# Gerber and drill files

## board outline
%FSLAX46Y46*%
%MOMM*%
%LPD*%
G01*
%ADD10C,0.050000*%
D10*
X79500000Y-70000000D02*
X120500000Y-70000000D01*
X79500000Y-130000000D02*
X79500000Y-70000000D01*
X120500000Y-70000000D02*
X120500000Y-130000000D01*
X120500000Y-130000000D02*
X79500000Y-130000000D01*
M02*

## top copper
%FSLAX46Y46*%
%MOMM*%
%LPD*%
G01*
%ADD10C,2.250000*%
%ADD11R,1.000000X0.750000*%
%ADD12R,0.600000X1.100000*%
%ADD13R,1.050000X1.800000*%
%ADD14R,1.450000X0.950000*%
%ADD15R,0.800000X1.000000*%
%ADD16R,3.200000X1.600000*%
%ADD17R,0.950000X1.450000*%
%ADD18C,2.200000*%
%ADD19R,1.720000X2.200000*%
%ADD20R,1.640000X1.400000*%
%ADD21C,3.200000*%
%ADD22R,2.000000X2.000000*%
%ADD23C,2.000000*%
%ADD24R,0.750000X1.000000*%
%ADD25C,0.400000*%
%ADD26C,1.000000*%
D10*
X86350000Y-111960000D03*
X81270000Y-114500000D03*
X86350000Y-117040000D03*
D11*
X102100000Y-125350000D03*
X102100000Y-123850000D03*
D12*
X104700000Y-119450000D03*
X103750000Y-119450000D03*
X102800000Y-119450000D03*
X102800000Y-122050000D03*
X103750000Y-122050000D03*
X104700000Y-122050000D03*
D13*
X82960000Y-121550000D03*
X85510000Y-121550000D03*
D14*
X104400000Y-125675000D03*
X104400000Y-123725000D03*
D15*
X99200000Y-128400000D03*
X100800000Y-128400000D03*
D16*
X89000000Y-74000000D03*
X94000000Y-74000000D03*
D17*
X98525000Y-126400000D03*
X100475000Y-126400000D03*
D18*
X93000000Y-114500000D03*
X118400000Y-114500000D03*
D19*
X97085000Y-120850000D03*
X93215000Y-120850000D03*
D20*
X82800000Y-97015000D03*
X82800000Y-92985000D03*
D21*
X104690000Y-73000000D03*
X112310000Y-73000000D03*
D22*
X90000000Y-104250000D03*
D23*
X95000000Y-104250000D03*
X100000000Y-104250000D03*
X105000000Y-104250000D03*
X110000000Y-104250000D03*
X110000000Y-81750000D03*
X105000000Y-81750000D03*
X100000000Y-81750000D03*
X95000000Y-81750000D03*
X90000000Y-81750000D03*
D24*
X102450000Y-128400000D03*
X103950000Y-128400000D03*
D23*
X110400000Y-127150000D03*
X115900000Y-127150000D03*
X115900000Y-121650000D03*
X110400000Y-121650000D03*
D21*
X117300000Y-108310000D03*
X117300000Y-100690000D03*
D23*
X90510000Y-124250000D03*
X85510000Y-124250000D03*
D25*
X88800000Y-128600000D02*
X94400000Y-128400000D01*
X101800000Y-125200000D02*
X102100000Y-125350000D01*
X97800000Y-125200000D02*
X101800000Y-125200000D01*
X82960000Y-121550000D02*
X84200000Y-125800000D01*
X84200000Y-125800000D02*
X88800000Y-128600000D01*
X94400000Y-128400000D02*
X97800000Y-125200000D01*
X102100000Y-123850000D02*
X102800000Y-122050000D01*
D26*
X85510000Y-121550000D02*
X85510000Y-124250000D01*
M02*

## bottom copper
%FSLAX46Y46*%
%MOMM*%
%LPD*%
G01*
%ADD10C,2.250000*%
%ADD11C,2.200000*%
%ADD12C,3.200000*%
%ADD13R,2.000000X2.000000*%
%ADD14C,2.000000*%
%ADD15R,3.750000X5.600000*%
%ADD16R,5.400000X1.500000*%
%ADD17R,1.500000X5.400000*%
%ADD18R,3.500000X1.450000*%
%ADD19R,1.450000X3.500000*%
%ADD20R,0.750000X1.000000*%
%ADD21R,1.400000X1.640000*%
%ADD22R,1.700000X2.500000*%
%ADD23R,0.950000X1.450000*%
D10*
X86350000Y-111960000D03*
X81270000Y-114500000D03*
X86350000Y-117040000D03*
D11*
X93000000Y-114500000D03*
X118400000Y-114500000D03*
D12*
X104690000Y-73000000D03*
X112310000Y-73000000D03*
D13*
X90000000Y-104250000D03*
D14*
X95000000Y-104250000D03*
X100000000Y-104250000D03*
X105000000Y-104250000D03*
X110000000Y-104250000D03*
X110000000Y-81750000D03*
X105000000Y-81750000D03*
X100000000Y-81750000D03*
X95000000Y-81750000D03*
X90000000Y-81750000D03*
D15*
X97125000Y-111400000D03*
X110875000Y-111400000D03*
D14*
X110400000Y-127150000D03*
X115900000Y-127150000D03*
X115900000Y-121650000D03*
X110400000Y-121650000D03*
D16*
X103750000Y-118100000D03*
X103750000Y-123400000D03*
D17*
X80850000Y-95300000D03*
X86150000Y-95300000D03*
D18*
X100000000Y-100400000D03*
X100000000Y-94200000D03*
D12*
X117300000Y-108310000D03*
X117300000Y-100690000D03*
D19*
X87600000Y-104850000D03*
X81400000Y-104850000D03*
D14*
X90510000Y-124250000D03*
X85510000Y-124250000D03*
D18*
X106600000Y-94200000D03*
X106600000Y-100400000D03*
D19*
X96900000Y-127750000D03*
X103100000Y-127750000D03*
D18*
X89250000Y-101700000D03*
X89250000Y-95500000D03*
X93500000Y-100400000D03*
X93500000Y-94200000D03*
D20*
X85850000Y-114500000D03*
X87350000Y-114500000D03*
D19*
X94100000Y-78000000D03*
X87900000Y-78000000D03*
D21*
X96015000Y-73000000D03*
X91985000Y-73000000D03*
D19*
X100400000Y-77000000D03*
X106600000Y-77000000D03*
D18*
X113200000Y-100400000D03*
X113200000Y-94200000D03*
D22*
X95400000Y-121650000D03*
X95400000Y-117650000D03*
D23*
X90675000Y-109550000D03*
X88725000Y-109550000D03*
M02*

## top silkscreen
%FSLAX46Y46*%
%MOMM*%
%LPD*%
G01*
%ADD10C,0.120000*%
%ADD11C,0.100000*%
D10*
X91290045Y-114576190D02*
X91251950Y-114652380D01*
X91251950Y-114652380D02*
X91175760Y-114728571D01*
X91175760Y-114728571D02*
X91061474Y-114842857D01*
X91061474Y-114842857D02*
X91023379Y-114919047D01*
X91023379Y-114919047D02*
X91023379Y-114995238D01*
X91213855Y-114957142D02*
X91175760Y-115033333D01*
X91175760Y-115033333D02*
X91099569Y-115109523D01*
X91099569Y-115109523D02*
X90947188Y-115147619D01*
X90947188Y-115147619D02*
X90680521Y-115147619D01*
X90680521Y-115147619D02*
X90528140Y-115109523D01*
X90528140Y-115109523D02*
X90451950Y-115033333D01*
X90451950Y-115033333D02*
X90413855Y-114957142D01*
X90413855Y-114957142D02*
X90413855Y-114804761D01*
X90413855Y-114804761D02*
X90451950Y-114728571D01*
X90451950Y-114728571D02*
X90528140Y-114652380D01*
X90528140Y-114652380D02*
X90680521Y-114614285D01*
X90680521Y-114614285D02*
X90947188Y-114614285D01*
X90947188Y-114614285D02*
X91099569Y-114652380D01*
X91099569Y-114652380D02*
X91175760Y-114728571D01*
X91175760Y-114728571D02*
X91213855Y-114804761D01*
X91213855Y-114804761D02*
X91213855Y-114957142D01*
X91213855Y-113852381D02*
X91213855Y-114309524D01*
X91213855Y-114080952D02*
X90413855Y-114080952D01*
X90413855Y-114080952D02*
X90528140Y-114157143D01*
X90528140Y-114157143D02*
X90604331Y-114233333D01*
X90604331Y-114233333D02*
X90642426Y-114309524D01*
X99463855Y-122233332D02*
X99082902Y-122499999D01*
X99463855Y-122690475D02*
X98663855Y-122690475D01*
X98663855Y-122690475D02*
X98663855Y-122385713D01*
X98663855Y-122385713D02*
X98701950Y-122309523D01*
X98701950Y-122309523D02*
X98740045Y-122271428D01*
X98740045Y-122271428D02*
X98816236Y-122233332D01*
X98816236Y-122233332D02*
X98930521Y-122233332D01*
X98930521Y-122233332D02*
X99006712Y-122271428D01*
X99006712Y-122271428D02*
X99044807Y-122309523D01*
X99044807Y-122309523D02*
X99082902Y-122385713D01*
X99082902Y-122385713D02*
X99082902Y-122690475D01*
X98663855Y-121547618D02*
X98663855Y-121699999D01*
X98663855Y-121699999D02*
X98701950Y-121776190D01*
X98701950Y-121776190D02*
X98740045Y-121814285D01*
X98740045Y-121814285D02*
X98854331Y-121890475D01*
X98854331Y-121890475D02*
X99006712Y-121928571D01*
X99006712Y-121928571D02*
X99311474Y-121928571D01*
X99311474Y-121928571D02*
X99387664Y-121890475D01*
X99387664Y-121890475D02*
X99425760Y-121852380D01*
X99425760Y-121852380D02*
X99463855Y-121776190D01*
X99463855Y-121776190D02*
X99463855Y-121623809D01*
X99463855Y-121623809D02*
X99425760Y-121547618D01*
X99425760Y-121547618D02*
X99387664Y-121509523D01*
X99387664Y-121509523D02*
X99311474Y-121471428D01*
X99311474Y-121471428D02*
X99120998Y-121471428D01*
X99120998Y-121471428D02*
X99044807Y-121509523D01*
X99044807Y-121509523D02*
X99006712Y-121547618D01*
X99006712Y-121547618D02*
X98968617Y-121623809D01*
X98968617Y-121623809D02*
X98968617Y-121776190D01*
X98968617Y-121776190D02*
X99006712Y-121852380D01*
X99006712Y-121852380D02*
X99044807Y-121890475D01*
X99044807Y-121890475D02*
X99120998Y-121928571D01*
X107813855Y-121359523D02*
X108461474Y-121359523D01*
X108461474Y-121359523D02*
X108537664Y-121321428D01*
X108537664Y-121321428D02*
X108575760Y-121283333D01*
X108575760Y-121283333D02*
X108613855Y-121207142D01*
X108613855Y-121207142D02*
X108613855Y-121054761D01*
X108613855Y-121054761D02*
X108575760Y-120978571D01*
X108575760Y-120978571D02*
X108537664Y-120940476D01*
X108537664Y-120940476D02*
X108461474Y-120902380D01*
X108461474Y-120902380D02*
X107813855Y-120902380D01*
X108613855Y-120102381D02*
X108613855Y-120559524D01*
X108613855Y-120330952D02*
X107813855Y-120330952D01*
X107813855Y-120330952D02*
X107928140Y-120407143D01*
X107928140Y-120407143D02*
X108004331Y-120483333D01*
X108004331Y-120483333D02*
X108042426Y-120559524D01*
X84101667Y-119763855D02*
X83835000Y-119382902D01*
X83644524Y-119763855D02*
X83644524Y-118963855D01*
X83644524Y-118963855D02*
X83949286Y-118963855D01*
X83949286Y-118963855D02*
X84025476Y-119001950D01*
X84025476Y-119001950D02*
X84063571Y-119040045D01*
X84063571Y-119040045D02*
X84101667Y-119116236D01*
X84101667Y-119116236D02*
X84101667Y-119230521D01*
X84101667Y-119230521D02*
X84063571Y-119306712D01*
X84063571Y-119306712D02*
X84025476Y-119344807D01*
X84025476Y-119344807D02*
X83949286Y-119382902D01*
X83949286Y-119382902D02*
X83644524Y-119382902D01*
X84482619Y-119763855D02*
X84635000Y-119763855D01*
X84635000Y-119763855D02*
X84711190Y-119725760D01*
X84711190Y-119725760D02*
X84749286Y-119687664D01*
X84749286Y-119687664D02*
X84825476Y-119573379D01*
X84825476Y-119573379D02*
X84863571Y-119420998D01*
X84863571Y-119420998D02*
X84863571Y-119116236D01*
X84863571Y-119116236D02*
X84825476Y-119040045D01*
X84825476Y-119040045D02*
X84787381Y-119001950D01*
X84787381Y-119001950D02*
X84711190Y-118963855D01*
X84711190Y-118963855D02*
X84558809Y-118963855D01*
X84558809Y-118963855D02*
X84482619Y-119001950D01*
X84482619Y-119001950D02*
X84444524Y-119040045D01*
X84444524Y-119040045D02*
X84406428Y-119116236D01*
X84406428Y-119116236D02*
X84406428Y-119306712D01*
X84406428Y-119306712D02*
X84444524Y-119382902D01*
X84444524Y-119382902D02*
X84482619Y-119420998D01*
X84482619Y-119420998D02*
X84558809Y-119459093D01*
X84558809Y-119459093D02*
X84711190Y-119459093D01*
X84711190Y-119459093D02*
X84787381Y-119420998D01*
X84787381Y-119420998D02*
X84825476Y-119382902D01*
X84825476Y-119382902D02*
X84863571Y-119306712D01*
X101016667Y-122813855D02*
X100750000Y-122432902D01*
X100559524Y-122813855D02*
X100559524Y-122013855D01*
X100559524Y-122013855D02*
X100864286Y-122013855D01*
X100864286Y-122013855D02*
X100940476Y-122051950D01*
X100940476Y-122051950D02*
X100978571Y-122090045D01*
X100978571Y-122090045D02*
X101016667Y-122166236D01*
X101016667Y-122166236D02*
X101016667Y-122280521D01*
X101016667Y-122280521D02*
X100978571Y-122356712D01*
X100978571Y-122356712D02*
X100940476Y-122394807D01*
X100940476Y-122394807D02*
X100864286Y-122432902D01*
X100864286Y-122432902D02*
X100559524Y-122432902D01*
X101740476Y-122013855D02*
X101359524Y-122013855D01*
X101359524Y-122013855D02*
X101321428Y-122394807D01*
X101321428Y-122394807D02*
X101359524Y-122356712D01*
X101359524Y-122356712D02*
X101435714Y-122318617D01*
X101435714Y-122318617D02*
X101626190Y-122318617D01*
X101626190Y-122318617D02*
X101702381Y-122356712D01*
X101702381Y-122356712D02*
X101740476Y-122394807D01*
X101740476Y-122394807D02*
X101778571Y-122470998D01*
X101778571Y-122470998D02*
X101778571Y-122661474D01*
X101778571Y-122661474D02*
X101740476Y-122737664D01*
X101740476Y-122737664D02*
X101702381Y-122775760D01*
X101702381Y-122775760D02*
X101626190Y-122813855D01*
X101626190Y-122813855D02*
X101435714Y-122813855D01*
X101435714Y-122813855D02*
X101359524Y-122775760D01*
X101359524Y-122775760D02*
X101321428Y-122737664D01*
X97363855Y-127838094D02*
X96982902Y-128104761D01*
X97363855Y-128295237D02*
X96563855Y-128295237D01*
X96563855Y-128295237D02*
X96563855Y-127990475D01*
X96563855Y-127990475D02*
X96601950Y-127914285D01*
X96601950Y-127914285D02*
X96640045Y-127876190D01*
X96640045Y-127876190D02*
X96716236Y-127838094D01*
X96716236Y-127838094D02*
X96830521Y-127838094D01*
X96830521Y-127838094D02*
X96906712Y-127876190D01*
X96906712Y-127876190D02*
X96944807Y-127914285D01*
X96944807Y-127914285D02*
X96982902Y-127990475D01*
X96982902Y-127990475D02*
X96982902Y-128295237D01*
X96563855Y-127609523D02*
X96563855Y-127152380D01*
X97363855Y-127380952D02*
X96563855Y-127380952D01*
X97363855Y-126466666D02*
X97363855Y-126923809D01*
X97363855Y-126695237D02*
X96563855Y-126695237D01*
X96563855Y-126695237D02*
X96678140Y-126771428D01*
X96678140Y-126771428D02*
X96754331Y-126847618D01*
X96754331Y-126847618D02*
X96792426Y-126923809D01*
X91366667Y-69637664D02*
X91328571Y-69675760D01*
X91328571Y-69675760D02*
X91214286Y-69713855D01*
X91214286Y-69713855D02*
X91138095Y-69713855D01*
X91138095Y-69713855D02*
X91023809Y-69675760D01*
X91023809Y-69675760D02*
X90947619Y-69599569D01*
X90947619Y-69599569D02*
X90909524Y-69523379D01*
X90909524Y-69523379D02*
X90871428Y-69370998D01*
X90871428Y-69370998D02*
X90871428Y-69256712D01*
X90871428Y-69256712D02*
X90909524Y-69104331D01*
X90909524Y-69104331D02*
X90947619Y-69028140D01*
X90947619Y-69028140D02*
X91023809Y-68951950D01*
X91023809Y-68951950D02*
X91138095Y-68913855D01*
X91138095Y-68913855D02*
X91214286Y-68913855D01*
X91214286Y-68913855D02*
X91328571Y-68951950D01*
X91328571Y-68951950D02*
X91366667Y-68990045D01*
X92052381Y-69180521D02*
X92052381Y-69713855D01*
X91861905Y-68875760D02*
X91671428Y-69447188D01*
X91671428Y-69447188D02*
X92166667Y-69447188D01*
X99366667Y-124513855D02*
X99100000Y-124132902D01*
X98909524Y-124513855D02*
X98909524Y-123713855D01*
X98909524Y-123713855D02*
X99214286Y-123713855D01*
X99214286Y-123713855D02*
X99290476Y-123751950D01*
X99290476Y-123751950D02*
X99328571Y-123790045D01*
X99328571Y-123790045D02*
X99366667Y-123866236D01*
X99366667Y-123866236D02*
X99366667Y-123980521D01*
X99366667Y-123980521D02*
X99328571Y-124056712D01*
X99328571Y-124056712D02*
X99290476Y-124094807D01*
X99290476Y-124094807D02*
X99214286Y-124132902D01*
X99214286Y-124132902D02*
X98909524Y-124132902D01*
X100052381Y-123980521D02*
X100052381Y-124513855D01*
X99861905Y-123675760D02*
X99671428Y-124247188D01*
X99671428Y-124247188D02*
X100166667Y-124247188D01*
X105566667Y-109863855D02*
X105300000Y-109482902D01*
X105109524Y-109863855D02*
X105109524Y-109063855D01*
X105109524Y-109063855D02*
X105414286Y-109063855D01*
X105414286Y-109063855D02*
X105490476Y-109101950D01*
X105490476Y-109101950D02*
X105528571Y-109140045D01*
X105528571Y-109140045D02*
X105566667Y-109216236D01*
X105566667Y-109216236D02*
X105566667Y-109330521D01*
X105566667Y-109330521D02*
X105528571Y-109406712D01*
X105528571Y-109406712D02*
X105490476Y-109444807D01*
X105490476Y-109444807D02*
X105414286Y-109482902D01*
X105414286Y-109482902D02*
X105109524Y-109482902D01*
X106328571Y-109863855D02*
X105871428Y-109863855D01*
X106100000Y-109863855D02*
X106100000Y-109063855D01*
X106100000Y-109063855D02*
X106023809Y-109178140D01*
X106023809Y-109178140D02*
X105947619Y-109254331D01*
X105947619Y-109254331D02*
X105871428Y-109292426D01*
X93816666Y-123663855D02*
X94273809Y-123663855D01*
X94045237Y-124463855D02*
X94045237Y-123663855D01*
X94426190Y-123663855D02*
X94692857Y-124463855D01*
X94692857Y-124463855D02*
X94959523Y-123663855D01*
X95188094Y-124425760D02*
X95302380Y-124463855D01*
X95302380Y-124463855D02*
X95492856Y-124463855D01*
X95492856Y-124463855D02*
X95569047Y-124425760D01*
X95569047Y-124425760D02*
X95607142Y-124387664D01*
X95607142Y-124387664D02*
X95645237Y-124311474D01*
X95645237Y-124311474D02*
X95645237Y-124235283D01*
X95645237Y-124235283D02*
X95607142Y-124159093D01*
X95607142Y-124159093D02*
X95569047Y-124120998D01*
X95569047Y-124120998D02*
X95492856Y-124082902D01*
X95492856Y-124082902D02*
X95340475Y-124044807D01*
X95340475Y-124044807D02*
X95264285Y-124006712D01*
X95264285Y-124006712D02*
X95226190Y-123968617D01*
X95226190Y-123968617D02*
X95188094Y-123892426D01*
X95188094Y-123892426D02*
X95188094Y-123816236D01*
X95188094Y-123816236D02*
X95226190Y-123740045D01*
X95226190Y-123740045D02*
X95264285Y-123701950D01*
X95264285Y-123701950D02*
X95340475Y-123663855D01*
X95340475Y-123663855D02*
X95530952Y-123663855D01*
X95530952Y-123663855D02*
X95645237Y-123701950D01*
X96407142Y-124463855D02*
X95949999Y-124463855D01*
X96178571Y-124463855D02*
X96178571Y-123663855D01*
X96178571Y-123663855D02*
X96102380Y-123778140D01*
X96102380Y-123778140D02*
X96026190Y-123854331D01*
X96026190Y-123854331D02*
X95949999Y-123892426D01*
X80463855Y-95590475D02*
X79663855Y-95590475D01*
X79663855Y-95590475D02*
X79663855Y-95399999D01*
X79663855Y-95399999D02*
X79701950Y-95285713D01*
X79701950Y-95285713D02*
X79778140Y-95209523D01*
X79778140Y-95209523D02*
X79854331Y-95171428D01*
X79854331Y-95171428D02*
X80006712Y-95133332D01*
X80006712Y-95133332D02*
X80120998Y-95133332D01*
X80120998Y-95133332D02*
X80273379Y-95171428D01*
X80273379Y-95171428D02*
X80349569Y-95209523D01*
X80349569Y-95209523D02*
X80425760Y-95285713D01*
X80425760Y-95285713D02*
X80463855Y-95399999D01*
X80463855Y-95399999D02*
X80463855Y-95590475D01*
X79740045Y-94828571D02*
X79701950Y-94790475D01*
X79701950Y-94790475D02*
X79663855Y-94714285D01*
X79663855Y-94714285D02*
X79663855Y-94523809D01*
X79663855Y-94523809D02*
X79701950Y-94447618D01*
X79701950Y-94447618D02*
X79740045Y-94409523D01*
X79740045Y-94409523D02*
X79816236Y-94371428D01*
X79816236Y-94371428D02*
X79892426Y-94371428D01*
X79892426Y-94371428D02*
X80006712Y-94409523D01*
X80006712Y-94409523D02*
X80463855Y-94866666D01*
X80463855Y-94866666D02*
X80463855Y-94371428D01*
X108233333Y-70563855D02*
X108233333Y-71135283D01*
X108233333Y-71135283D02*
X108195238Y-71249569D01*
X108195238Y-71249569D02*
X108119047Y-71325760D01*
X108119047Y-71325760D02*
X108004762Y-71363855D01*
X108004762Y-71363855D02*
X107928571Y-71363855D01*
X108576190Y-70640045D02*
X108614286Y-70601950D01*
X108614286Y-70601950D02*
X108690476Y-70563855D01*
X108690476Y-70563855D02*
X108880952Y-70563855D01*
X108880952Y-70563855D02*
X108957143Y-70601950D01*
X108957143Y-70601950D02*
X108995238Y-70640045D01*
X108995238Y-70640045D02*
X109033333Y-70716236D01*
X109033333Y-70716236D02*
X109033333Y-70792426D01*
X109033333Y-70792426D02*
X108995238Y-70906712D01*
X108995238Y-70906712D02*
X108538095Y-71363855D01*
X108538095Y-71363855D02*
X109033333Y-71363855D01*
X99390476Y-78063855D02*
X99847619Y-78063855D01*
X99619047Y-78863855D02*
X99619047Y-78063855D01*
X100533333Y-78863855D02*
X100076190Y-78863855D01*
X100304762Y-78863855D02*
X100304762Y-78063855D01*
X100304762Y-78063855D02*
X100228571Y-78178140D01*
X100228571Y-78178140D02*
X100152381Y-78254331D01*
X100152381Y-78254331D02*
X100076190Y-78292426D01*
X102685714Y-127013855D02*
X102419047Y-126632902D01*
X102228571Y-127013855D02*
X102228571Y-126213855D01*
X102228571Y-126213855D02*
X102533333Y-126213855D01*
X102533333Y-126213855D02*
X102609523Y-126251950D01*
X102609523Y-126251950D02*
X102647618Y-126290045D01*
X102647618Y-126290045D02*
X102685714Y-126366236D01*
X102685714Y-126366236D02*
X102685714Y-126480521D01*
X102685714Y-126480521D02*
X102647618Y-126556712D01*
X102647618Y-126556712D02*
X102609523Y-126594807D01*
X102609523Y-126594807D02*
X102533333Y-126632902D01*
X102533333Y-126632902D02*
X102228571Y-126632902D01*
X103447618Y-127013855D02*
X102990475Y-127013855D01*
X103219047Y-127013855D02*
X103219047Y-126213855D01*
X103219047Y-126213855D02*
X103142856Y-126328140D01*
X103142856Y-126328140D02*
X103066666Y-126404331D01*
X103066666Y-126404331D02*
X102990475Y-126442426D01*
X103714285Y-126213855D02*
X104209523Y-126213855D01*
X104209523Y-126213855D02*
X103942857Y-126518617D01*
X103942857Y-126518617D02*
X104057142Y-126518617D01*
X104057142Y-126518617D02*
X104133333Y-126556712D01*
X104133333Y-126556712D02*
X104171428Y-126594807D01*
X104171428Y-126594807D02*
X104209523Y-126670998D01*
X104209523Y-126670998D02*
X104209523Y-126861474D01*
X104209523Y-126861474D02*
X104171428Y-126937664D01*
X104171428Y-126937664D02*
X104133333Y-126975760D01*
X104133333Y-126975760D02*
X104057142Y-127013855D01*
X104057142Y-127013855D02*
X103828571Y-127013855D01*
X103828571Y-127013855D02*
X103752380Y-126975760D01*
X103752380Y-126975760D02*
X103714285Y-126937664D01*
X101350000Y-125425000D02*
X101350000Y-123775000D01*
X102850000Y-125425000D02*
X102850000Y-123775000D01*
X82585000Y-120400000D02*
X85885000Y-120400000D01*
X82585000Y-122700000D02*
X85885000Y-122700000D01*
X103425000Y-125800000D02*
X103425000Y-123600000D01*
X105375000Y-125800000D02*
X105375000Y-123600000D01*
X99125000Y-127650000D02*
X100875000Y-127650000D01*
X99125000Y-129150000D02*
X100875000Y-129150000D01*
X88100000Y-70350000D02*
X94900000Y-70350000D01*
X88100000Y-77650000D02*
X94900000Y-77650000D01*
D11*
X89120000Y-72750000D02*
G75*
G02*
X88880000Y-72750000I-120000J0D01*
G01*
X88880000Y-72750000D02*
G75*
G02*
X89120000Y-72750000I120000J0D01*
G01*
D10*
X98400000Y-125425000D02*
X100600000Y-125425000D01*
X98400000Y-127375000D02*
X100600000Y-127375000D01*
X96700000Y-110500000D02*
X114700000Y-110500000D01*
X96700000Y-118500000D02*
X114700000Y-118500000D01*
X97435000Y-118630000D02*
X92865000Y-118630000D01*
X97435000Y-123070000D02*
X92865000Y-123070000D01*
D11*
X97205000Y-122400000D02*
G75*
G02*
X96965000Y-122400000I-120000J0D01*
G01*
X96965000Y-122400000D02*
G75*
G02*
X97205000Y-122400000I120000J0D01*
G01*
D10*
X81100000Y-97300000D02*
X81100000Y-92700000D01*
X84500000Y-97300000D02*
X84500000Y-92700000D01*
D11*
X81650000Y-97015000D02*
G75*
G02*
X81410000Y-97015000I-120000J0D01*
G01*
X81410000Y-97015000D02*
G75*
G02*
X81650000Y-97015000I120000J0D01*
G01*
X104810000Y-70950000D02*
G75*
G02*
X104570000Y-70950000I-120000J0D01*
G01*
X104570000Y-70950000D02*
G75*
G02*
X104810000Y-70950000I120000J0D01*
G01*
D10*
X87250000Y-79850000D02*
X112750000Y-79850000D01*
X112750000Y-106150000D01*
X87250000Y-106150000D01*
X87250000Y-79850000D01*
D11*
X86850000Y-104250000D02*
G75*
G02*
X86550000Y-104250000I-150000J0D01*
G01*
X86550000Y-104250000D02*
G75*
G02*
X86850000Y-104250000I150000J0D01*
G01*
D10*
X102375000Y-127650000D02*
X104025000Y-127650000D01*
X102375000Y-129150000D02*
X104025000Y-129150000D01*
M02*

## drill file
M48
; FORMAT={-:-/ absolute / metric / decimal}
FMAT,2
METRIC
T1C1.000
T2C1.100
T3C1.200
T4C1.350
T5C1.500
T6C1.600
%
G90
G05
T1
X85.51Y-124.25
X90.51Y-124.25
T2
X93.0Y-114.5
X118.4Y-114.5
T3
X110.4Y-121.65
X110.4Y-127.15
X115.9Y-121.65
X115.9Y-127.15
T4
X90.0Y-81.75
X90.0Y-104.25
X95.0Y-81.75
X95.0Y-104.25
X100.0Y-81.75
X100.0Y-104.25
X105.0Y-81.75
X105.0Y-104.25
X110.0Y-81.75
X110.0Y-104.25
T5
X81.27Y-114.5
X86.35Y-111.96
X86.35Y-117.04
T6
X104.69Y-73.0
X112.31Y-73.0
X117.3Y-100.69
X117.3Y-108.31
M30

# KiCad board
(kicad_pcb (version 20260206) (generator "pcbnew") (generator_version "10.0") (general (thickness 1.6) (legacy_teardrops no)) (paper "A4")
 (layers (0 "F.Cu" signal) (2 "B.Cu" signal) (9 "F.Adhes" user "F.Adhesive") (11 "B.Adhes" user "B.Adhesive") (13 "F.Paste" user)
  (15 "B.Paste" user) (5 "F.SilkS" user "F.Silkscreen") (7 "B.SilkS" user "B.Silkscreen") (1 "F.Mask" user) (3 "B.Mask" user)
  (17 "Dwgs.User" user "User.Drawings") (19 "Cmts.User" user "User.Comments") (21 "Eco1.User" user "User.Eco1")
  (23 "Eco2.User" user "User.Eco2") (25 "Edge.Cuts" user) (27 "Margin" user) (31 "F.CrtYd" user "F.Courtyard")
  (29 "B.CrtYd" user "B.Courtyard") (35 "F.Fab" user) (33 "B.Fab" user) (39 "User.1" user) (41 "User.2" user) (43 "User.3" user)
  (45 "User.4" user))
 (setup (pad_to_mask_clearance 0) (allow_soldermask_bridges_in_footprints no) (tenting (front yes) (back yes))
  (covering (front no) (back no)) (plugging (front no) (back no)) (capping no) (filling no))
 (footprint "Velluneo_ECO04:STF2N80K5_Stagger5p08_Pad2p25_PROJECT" (layer "F.Cu") (at 86.35 114.5 -90)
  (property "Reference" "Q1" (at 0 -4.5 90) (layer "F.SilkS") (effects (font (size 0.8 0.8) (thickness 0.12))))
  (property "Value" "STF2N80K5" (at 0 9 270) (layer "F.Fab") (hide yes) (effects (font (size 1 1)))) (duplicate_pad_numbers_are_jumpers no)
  (pad "1" thru_hole circle (at -2.54 0 270) (size 2.25 2.25) (drill 1.5) (layers "*.Cu" "*.Mask") (remove_unused_layers no) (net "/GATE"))
  (pad "2" thru_hole circle (at 0 5.08 270) (size 2.25 2.25) (drill 1.5) (layers "*.Cu" "*.Mask") (remove_unused_layers no) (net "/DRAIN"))
  (pad "3" thru_hole circle (at 2.54 0 270) (size 2.25 2.25) (drill 1.5) (layers "*.Cu" "*.Mask") (remove_unused_layers no) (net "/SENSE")))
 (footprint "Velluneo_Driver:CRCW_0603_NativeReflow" (layer "F.Cu") (at 102.1 124.6 90)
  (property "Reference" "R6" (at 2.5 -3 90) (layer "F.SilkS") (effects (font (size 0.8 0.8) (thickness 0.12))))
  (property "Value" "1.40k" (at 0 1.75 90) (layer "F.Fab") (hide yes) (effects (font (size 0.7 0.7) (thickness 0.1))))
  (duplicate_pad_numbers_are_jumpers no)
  (fp_line (start -0.825 -0.75) (end 0.825 -0.75) (stroke (width 0.12) (type default)) (layer "F.SilkS"))
  (fp_line (start -0.825 0.75) (end 0.825 0.75) (stroke (width 0.12) (type default)) (layer "F.SilkS"))
  (pad "1" smd rect (at -0.75 0 90) (size 0.75 1) (layers "F.Cu" "F.Mask" "F.Paste") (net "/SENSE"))
  (pad "2" smd rect (at 0.75 0 90) (size 0.75 1) (layers "F.Cu" "F.Mask" "F.Paste") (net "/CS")))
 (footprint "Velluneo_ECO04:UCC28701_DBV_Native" (layer "F.Cu") (at 103.75 120.75 -90)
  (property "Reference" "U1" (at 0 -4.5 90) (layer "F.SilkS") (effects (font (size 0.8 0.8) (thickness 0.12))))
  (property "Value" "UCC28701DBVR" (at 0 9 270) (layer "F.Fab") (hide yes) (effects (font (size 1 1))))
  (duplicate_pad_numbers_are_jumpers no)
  (pad "1" smd rect (at -1.3 -0.95 270) (size 1.1 0.6) (layers "F.Cu" "F.Mask" "F.Paste") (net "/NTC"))
  (pad "2" smd rect (at -1.3 0 270) (size 1.1 0.6) (layers "F.Cu" "F.Mask" "F.Paste") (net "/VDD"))
  (pad "3" smd rect (at -1.3 0.95 270) (size 1.1 0.6) (layers "F.Cu" "F.Mask" "F.Paste") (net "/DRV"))
  (pad "4" smd rect (at 1.3 0.95 270) (size 1.1 0.6) (layers "F.Cu" "F.Mask" "F.Paste") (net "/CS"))
  (pad "5" smd rect (at 1.3 0 270) (size 1.1 0.6) (layers "F.Cu" "F.Mask" "F.Paste") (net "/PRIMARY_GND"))
  (pad "6" smd rect (at 1.3 -0.95 270) (size 1.1 0.6) (layers "F.Cu" "F.Mask" "F.Paste") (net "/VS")))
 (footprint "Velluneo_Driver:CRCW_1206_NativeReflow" (layer "F.Cu") (at 84.235 121.55)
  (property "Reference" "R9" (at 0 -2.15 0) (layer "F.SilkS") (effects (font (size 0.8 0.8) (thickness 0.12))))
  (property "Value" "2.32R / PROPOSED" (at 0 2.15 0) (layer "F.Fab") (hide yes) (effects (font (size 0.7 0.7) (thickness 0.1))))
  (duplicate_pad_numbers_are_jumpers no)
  (fp_line (start -1.65 -1.15) (end 1.65 -1.15) (stroke (width 0.12) (type default)) (layer "F.SilkS"))
  (fp_line (start -1.65 1.15) (end 1.65 1.15) (stroke (width 0.12) (type default)) (layer "F.SilkS"))
  (pad "1" smd rect (at -1.275 0) (size 1.05 1.8) (layers "F.Cu" "F.Mask" "F.Paste") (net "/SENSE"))
  (pad "2" smd rect (at 1.275 0) (size 1.05 1.8) (layers "F.Cu" "F.Mask" "F.Paste") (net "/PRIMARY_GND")))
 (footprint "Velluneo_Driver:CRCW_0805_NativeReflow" (layer "F.Cu") (at 104.4 124.7 90)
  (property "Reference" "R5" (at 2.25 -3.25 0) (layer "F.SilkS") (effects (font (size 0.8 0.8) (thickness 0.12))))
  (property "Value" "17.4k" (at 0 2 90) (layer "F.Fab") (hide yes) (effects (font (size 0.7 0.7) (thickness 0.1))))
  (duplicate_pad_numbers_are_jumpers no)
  (fp_line (start -1.1 -0.975) (end 1.1 -0.975) (stroke (width 0.12) (type default)) (layer "F.SilkS"))
  (fp_line (start -1.1 0.975) (end 1.1 0.975) (stroke (width 0.12) (type default)) (layer "F.SilkS"))
  (pad "1" smd rect (at -0.975 0 90) (size 0.95 1.45) (layers "F.Cu" "F.Mask" "F.Paste") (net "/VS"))
  (pad "2" smd rect (at 0.975 0 90) (size 0.95 1.45) (layers "F.Cu" "F.Mask" "F.Paste") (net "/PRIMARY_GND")))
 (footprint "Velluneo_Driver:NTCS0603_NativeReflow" (layer "F.Cu") (at 100 128.4)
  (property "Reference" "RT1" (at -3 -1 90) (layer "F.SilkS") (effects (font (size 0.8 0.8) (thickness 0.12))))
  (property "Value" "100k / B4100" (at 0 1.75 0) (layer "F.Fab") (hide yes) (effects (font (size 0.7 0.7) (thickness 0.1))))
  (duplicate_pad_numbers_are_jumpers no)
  (fp_line (start -0.875 -0.75) (end 0.875 -0.75) (stroke (width 0.12) (type default)) (layer "F.SilkS"))
  (fp_line (start -0.875 0.75) (end 0.875 0.75) (stroke (width 0.12) (type default)) (layer "F.SilkS"))
  (pad "1" smd rect (at -0.8 0) (size 0.8 1) (layers "F.Cu" "F.Mask" "F.Paste") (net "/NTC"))
  (pad "2" smd rect (at 0.8 0) (size 0.8 1) (layers "F.Cu" "F.Mask" "F.Paste") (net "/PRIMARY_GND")))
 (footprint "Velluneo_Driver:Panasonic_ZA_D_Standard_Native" (layer "F.Cu") (at 91.5 74)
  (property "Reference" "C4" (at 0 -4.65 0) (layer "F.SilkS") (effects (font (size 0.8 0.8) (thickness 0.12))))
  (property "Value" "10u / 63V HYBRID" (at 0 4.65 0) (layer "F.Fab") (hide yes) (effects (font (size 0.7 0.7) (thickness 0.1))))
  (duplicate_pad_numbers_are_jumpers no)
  (fp_line (start -3.4 -3.65) (end 3.4 -3.65) (stroke (width 0.12) (type default)) (layer "F.SilkS"))
  (fp_line (start -3.4 3.65) (end 3.4 3.65) (stroke (width 0.12) (type default)) (layer "F.SilkS"))
  (fp_circle (center -2.5 -1.25) (end -2.38 -1.25) (stroke (width 0.1) (type default)) (fill no) (layer "F.SilkS"))
  (pad "1" smd rect (at -2.5 0) (size 3.2 1.6) (layers "F.Cu" "F.Mask" "F.Paste") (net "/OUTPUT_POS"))
  (pad "2" smd rect (at 2.5 0) (size 3.2 1.6) (layers "F.Cu" "F.Mask" "F.Paste") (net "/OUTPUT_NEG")))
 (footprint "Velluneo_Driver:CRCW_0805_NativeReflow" (layer "F.Cu") (at 99.5 126.4)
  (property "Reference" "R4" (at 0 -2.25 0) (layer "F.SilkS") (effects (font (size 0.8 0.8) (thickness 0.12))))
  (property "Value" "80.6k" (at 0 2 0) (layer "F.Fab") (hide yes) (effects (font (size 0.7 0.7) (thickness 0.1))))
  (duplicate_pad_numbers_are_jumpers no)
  (fp_line (start -1.1 -0.975) (end 1.1 -0.975) (stroke (width 0.12) (type default)) (layer "F.SilkS"))
  (fp_line (start -1.1 0.975) (end 1.1 0.975) (stroke (width 0.12) (type default)) (layer "F.SilkS"))
  (pad "1" smd rect (at -0.975 0) (size 0.95 1.45) (layers "F.Cu" "F.Mask" "F.Paste") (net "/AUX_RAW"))
  (pad "2" smd rect (at 0.975 0) (size 0.95 1.45) (layers "F.Cu" "F.Mask" "F.Paste") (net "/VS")))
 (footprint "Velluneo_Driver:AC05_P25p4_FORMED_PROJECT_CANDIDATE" (layer "F.Cu") (at 105.7 114.5)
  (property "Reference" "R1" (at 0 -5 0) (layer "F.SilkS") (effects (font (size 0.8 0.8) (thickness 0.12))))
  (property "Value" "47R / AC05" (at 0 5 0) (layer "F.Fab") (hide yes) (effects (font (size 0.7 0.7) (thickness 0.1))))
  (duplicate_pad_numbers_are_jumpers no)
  (fp_line (start -9 -4) (end 9 -4) (stroke (width 0.12) (type default)) (layer "F.SilkS"))
  (fp_line (start -9 4) (end 9 4) (stroke (width 0.12) (type default)) (layer "F.SilkS"))
  (pad "1" thru_hole circle (at -12.7 0) (size 2.2 2.2) (drill 1.1) (layers "*.Cu" "*.Mask") (remove_unused_layers no) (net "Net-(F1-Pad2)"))
  (pad "2" thru_hole circle (at 12.7 0) (size 2.2 2.2) (drill 1.1) (layers "*.Cu" "*.Mask") (remove_unused_layers no)
   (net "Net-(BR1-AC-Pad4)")))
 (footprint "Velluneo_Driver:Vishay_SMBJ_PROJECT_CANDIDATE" (layer "F.Cu") (at 95.15 120.85 180)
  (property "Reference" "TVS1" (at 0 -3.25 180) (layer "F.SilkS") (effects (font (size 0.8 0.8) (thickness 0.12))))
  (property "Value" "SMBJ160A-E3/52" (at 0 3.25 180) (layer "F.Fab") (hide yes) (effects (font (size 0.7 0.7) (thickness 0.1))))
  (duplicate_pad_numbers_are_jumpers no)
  (fp_line (start -2.285 2.22) (end 2.285 2.22) (stroke (width 0.12) (type default)) (layer "F.SilkS"))
  (fp_line (start -2.285 -2.22) (end 2.285 -2.22) (stroke (width 0.12) (type default)) (layer "F.SilkS"))
  (fp_circle (center -1.935 -1.55) (end -1.815 -1.55) (stroke (width 0.1) (type default)) (fill no) (layer "F.SilkS"))
  (pad "1" smd rect (at -1.935 0 180) (size 1.72 2.2) (layers "F.Cu" "F.Mask" "F.Paste") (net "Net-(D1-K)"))
  (pad "2" smd rect (at 1.935 0 180) (size 1.72 2.2) (layers "F.Cu" "F.Mask" "F.Paste") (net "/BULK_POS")))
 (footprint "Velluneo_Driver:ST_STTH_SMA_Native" (layer "F.Cu") (at 82.8 95 90)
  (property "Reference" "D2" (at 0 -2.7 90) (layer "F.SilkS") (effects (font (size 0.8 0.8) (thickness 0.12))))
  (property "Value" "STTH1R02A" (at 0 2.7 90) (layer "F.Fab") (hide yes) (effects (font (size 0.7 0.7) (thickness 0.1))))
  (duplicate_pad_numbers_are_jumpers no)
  (fp_line (start -2.3 -1.7) (end 2.3 -1.7) (stroke (width 0.12) (type default)) (layer "F.SilkS"))
  (fp_line (start -2.3 1.7) (end 2.3 1.7) (stroke (width 0.12) (type default)) (layer "F.SilkS"))
  (fp_circle (center -2.015 -1.27) (end -1.895 -1.27) (stroke (width 0.1) (type default)) (fill no) (layer "F.SilkS"))
  (pad "1" smd rect (at -2.015 0 90) (size 1.4 1.64) (layers "F.Cu" "F.Mask" "F.Paste") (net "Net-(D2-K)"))
  (pad "2" smd rect (at 2.015 0 90) (size 1.4 1.64) (layers "F.Cu" "F.Mask" "F.Paste") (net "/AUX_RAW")))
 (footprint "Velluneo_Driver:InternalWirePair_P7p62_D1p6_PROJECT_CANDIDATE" (layer "F.Cu") (at 108.5 73)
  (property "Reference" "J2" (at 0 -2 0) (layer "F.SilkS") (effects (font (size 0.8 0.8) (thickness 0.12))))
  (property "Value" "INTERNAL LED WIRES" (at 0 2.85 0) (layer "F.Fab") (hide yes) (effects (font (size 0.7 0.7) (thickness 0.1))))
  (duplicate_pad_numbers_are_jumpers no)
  (fp_circle (center -3.81 -2.05) (end -3.69 -2.05) (stroke (width 0.1) (type default)) (fill no) (layer "F.SilkS"))
  (pad "1" thru_hole circle (at -3.81 0) (size 3.2 3.2) (drill 1.6) (layers "*.Cu" "*.Mask") (remove_unused_layers no) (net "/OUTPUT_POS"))
  (pad "2" thru_hole circle (at 3.81 0) (size 3.2 3.2) (drill 1.6) (layers "*.Cu" "*.Mask") (remove_unused_layers no) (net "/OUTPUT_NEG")))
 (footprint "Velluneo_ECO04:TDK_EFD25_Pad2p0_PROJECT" (layer "F.Cu") (at 100 93)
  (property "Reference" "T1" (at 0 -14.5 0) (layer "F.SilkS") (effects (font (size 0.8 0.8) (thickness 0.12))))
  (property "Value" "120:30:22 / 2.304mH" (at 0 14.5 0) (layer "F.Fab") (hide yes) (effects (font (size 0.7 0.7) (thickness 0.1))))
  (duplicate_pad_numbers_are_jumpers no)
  (fp_rect (start -12.75 -13.15) (end 12.75 13.15) (stroke (width 0.12) (type default)) (fill no) (layer "F.SilkS"))
  (fp_circle (center -13.3 11.25) (end -13.15 11.25) (stroke (width 0.1) (type default)) (fill no) (layer "F.SilkS"))
  (pad "1" thru_hole rect (at -10 11.25) (size 2 2) (drill 1.35) (layers "*.Cu" "*.Mask") (remove_unused_layers no) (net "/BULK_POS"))
  (pad "2" thru_hole circle (at -5 11.25) (size 2 2) (drill 1.35) (layers "*.Cu" "*.Mask") (remove_unused_layers no) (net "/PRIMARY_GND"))
  (pad "3" thru_hole circle (at 0 11.25) (size 2 2) (drill 1.35) (layers "*.Cu" "*.Mask") (remove_unused_layers no)
   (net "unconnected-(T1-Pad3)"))
  (pad "4" thru_hole circle (at 5 11.25) (size 2 2) (drill 1.35) (layers "*.Cu" "*.Mask") (remove_unused_layers no) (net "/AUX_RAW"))
  (pad "5" thru_hole circle (at 10 11.25) (size 2 2) (drill 1.35) (layers "*.Cu" "*.Mask") (remove_unused_layers no) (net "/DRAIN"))
  (pad "6" thru_hole circle (at 10 -11.25) (size 2 2) (drill 1.35) (layers "*.Cu" "*.Mask") (remove_unused_layers no) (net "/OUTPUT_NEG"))
  (pad "7" thru_hole circle (at 5 -11.25) (size 2 2) (drill 1.35) (layers "*.Cu" "*.Mask") (remove_unused_layers no)
   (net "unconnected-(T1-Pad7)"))
  (pad "8" thru_hole circle (at 0 -11.25) (size 2 2) (drill 1.35) (layers "*.Cu" "*.Mask") (remove_unused_layers no)
   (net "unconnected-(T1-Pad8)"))
  (pad "9" thru_hole circle (at -5 -11.25) (size 2 2) (drill 1.35) (layers "*.Cu" "*.Mask") (remove_unused_layers no)
   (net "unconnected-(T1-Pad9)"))
  (pad "10" thru_hole circle (at -10 -11.25) (size 2 2) (drill 1.35) (layers "*.Cu" "*.Mask") (remove_unused_layers no)
   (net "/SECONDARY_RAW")))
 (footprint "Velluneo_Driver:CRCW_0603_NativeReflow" (layer "F.Cu") (at 103.2 128.4)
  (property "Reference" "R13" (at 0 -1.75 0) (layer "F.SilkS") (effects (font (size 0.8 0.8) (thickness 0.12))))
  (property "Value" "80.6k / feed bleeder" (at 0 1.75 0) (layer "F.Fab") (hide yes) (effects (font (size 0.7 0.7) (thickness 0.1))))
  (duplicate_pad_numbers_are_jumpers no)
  (fp_line (start -0.825 -0.75) (end 0.825 -0.75) (stroke (width 0.12) (type default)) (layer "F.SilkS"))
  (fp_line (start -0.825 0.75) (end 0.825 0.75) (stroke (width 0.12) (type default)) (layer "F.SilkS"))
  (pad "1" smd rect (at -0.75 0) (size 0.75 1) (layers "F.Cu" "F.Mask" "F.Paste") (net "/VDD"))
  (pad "2" smd rect (at 0.75 0) (size 0.75 1) (layers "F.Cu" "F.Mask" "F.Paste") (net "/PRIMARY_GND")))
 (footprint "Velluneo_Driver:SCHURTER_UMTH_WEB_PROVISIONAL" (layer "B.Cu") (at 104 111.4)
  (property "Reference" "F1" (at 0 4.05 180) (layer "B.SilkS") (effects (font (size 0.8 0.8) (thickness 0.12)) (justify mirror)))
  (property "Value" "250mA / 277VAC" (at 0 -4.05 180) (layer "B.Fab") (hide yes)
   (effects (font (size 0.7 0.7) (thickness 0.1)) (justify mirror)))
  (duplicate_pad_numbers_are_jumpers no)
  (pad "1" smd rect (at -6.875 0) (size 3.75 5.6) (layers "B.Cu" "B.Mask" "B.Paste") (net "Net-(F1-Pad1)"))
  (pad "2" smd rect (at 6.875 0) (size 3.75 5.6) (layers "B.Cu" "B.Mask" "B.Paste") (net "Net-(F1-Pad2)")))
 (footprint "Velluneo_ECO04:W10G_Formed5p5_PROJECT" (layer "B.Cu") (at 113.15 124.4)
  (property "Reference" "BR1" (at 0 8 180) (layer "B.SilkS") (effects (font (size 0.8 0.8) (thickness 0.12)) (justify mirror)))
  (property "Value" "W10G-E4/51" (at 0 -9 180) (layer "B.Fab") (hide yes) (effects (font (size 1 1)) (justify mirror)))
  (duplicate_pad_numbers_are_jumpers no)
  (pad "1" thru_hole circle (at -2.75 2.75) (size 2 2) (drill 1.2) (layers "*.Cu" "*.Mask") (remove_unused_layers no) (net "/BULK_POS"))
  (pad "2" thru_hole circle (at 2.75 2.75) (size 2 2) (drill 1.2) (layers "*.Cu" "*.Mask") (remove_unused_layers no)
   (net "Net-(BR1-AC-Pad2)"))
  (pad "3" thru_hole circle (at 2.75 -2.75) (size 2 2) (drill 1.2) (layers "*.Cu" "*.Mask") (remove_unused_layers no) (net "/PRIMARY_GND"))
  (pad "4" thru_hole circle (at -2.75 -2.75) (size 2 2) (drill 1.2) (layers "*.Cu" "*.Mask") (remove_unused_layers no)
   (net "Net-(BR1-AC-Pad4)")))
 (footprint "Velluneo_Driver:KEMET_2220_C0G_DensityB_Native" (layer "B.Cu") (at 103.75 120.75 -90)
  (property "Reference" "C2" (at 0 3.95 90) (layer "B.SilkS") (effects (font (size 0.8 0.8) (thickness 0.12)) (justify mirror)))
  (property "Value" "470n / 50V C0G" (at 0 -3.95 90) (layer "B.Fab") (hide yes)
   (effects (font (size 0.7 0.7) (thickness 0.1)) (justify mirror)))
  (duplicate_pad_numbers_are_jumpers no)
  (pad "1" smd rect (at -2.65 0 270) (size 1.5 5.4) (layers "B.Cu" "B.Mask" "B.Paste") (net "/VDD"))
  (pad "2" smd rect (at 2.65 0 270) (size 1.5 5.4) (layers "B.Cu" "B.Mask" "B.Paste") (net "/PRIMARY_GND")))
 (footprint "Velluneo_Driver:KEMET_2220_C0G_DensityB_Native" (layer "B.Cu") (at 83.5 95.3)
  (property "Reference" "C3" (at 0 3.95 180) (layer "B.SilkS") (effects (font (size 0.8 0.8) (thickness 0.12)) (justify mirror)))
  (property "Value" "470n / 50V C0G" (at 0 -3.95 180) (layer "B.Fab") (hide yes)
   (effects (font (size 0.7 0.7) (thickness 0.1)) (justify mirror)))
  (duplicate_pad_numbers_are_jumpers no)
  (pad "1" smd rect (at -2.65 0) (size 1.5 5.4) (layers "B.Cu" "B.Mask" "B.Paste") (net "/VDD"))
  (pad "2" smd rect (at 2.65 0) (size 1.5 5.4) (layers "B.Cu" "B.Mask" "B.Paste") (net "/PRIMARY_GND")))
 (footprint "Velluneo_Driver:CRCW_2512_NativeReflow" (layer "B.Cu") (at 100 97.3 90)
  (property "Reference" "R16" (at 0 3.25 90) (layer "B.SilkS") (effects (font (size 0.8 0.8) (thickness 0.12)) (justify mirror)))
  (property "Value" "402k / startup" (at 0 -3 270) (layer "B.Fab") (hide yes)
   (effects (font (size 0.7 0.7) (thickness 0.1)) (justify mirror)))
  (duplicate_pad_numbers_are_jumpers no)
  (pad "1" smd rect (at -3.1 0 90) (size 1.45 3.5) (layers "B.Cu" "B.Mask" "B.Paste") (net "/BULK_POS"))
  (pad "2" smd rect (at 3.1 0 90) (size 1.45 3.5) (layers "B.Cu" "B.Mask" "B.Paste") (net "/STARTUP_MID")))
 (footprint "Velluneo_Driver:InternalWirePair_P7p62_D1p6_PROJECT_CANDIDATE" (layer "B.Cu") (at 117.3 104.5 90)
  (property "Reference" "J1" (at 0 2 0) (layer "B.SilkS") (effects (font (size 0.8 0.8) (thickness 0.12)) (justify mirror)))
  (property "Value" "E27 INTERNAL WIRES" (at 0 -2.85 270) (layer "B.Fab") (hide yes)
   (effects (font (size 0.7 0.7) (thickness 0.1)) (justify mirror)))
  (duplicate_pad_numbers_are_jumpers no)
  (pad "1" thru_hole circle (at -3.81 0 90) (size 3.2 3.2) (drill 1.6) (layers "*.Cu" "*.Mask") (remove_unused_layers no)
   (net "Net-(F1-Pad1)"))
  (pad "2" thru_hole circle (at 3.81 0 90) (size 3.2 3.2) (drill 1.6) (layers "*.Cu" "*.Mask") (remove_unused_layers no)
   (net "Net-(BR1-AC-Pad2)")))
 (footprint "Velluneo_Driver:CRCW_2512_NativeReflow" (layer "B.Cu") (at 84.5 104.85 180)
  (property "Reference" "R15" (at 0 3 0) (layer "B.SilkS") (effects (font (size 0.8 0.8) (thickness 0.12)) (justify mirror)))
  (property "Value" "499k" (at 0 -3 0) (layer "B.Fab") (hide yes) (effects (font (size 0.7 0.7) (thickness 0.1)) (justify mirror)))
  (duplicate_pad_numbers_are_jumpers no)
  (pad "1" smd rect (at -3.1 0 180) (size 1.45 3.5) (layers "B.Cu" "B.Mask" "B.Paste") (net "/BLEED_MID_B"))
  (pad "2" smd rect (at 3.1 0 180) (size 1.45 3.5) (layers "B.Cu" "B.Mask" "B.Paste") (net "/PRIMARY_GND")))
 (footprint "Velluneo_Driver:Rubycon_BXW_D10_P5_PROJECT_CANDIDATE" (layer "B.Cu") (at 88.01 124.25 180)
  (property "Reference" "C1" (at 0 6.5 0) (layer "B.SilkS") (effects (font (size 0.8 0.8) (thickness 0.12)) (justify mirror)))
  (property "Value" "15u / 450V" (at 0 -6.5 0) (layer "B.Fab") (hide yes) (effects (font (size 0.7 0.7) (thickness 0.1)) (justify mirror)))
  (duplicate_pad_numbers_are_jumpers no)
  (pad "1" thru_hole circle (at -2.5 0 180) (size 2 2) (drill 1) (layers "*.Cu" "*.Mask") (remove_unused_layers no) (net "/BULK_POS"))
  (pad "2" thru_hole circle (at 2.5 0 180) (size 2 2) (drill 1) (layers "*.Cu" "*.Mask") (remove_unused_layers no) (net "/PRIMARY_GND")))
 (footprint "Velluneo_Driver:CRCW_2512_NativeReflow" (layer "B.Cu") (at 106.6 97.3 -90)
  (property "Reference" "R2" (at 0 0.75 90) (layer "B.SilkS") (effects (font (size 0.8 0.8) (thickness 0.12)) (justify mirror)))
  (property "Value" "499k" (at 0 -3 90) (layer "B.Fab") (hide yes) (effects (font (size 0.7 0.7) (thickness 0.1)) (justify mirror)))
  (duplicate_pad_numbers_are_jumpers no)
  (pad "1" smd rect (at -3.1 0 270) (size 1.45 3.5) (layers "B.Cu" "B.Mask" "B.Paste") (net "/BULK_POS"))
  (pad "2" smd rect (at 3.1 0 270) (size 1.45 3.5) (layers "B.Cu" "B.Mask" "B.Paste") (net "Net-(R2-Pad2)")))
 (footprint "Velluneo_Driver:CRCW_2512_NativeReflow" (layer "B.Cu") (at 100 127.75)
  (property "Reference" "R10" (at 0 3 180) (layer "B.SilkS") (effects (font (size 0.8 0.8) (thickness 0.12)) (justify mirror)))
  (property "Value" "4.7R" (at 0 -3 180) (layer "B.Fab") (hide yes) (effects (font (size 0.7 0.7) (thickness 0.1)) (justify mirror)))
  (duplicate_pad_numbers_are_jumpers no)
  (pad "1" smd rect (at -3.1 0) (size 1.45 3.5) (layers "B.Cu" "B.Mask" "B.Paste") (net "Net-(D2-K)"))
  (pad "2" smd rect (at 3.1 0) (size 1.45 3.5) (layers "B.Cu" "B.Mask" "B.Paste") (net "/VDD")))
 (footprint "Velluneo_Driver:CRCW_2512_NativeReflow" (layer "B.Cu") (at 89.25 98.6 90)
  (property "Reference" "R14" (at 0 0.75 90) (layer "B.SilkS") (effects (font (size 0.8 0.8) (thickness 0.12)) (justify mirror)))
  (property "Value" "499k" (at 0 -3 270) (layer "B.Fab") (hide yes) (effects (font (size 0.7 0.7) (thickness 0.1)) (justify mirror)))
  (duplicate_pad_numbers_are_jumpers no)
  (pad "1" smd rect (at -3.1 0 90) (size 1.45 3.5) (layers "B.Cu" "B.Mask" "B.Paste") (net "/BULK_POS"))
  (pad "2" smd rect (at 3.1 0 90) (size 1.45 3.5) (layers "B.Cu" "B.Mask" "B.Paste") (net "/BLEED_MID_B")))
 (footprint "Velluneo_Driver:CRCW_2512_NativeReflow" (layer "B.Cu") (at 93.5 97.3 90)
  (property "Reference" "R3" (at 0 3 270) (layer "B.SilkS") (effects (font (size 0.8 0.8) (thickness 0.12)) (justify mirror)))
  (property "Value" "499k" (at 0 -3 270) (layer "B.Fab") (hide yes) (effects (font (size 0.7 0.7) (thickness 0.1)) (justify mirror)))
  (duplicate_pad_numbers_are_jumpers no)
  (pad "1" smd rect (at -3.1 0 90) (size 1.45 3.5) (layers "B.Cu" "B.Mask" "B.Paste") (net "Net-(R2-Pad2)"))
  (pad "2" smd rect (at 3.1 0 90) (size 1.45 3.5) (layers "B.Cu" "B.Mask" "B.Paste") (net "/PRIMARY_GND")))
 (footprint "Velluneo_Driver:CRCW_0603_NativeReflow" (layer "B.Cu") (at 86.6 114.5)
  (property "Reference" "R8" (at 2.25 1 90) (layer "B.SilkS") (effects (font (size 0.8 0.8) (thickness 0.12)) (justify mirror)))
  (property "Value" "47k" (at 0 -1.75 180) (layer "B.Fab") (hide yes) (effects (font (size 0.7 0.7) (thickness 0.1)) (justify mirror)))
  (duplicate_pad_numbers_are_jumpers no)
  (pad "1" smd rect (at -0.75 0) (size 0.75 1) (layers "B.Cu" "B.Mask" "B.Paste") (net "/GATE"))
  (pad "2" smd rect (at 0.75 0) (size 0.75 1) (layers "B.Cu" "B.Mask" "B.Paste") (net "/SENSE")))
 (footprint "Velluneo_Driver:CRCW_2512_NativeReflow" (layer "B.Cu") (at 91 78 180)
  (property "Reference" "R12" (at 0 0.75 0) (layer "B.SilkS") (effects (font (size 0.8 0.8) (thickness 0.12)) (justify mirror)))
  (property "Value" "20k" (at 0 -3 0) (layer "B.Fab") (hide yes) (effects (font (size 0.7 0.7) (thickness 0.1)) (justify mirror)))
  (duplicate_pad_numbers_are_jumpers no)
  (pad "1" smd rect (at -3.1 0 180) (size 1.45 3.5) (layers "B.Cu" "B.Mask" "B.Paste") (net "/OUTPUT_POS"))
  (pad "2" smd rect (at 3.1 0 180) (size 1.45 3.5) (layers "B.Cu" "B.Mask" "B.Paste") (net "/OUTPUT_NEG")))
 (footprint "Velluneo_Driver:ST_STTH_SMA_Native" (layer "B.Cu") (at 94 73 180)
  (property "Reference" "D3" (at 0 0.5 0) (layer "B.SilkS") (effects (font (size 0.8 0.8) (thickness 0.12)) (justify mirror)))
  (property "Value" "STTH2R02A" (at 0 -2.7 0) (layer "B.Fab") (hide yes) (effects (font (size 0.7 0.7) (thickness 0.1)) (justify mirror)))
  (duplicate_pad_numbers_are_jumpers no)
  (pad "1" smd rect (at -2.015 0 180) (size 1.4 1.64) (layers "B.Cu" "B.Mask" "B.Paste") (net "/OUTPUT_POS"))
  (pad "2" smd rect (at 2.015 0 180) (size 1.4 1.64) (layers "B.Cu" "B.Mask" "B.Paste") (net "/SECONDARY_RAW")))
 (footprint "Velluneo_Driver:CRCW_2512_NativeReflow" (layer "B.Cu") (at 103.5 77)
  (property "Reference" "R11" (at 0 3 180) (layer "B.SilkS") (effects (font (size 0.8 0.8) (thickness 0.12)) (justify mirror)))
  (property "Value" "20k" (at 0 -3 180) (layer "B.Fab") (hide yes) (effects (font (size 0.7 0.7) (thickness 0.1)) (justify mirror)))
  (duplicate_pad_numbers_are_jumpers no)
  (pad "1" smd rect (at -3.1 0) (size 1.45 3.5) (layers "B.Cu" "B.Mask" "B.Paste") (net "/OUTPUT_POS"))
  (pad "2" smd rect (at 3.1 0) (size 1.45 3.5) (layers "B.Cu" "B.Mask" "B.Paste") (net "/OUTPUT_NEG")))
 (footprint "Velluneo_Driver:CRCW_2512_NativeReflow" (layer "B.Cu") (at 113.2 97.3 90)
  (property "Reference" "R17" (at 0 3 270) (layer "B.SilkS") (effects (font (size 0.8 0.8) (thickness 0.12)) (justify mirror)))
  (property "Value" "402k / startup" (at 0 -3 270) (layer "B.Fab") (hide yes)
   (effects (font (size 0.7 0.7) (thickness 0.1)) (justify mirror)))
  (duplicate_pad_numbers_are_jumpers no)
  (pad "1" smd rect (at -3.1 0 90) (size 1.45 3.5) (layers "B.Cu" "B.Mask" "B.Paste") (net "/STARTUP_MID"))
  (pad "2" smd rect (at 3.1 0 90) (size 1.45 3.5) (layers "B.Cu" "B.Mask" "B.Paste") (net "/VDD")))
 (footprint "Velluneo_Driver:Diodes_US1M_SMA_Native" (layer "B.Cu") (at 95.4 119.65 90)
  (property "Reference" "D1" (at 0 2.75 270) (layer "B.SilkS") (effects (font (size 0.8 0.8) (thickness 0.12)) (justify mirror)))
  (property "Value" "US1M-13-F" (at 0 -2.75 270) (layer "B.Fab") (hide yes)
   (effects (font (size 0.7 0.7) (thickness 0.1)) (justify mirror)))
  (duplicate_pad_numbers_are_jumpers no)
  (pad "1" smd rect (at -2 0 90) (size 2.5 1.7) (layers "B.Cu" "B.Mask" "B.Paste") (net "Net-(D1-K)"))
  (pad "2" smd rect (at 2 0 90) (size 2.5 1.7) (layers "B.Cu" "B.Mask" "B.Paste") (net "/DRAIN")))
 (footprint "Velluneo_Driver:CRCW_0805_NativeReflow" (layer "B.Cu") (at 89.7 109.55 180)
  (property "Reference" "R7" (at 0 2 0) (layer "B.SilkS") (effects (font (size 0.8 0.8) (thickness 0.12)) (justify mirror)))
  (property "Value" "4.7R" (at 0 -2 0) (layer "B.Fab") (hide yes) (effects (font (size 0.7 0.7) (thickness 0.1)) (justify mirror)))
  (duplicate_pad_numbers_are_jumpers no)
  (pad "1" smd rect (at -0.975 0 180) (size 0.95 1.45) (layers "B.Cu" "B.Mask" "B.Paste") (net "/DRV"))
  (pad "2" smd rect (at 0.975 0 180) (size 0.95 1.45) (layers "B.Cu" "B.Mask" "B.Paste") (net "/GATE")))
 (gr_line (start 79.5 70) (end 120.5 70) (stroke (width 0.05) (type default)) (layer "Edge.Cuts"))
 (gr_line (start 79.5 130) (end 79.5 70) (stroke (width 0.05) (type default)) (layer "Edge.Cuts"))
 (gr_line (start 120.5 70) (end 120.5 130) (stroke (width 0.05) (type default)) (layer "Edge.Cuts"))
 (gr_line (start 120.5 130) (end 79.5 130) (stroke (width 0.05) (type default)) (layer "Edge.Cuts"))
 (segment (start 88.8 128.6) (end 94.4 128.4) (width 0.4) (layer "F.Cu") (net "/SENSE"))
 (segment (start 101.8 125.2) (end 102.1 125.35) (width 0.4) (layer "F.Cu") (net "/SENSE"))
 (segment (start 97.8 125.2) (end 101.8 125.2) (width 0.4) (layer "F.Cu") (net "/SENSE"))
 (segment (start 82.96 121.55) (end 84.2 125.8) (width 0.4) (layer "F.Cu") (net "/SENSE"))
 (segment (start 84.2 125.8) (end 88.8 128.6) (width 0.4) (layer "F.Cu") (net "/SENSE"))
 (segment (start 94.4 128.4) (end 97.8 125.2) (width 0.4) (layer "F.Cu") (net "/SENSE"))
 (segment (start 102.1 123.85) (end 102.8 122.05) (width 0.4) (layer "F.Cu") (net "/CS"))
 (segment (start 85.51 121.55) (end 85.51 124.25) (width 1) (layer "F.Cu") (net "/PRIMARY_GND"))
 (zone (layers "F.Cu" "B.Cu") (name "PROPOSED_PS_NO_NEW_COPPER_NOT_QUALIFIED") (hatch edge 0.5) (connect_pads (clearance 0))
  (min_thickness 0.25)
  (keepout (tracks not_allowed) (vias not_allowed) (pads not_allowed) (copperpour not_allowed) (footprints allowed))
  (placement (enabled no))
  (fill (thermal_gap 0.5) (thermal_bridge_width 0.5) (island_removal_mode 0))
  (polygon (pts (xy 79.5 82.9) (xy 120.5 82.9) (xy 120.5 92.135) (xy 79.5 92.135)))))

